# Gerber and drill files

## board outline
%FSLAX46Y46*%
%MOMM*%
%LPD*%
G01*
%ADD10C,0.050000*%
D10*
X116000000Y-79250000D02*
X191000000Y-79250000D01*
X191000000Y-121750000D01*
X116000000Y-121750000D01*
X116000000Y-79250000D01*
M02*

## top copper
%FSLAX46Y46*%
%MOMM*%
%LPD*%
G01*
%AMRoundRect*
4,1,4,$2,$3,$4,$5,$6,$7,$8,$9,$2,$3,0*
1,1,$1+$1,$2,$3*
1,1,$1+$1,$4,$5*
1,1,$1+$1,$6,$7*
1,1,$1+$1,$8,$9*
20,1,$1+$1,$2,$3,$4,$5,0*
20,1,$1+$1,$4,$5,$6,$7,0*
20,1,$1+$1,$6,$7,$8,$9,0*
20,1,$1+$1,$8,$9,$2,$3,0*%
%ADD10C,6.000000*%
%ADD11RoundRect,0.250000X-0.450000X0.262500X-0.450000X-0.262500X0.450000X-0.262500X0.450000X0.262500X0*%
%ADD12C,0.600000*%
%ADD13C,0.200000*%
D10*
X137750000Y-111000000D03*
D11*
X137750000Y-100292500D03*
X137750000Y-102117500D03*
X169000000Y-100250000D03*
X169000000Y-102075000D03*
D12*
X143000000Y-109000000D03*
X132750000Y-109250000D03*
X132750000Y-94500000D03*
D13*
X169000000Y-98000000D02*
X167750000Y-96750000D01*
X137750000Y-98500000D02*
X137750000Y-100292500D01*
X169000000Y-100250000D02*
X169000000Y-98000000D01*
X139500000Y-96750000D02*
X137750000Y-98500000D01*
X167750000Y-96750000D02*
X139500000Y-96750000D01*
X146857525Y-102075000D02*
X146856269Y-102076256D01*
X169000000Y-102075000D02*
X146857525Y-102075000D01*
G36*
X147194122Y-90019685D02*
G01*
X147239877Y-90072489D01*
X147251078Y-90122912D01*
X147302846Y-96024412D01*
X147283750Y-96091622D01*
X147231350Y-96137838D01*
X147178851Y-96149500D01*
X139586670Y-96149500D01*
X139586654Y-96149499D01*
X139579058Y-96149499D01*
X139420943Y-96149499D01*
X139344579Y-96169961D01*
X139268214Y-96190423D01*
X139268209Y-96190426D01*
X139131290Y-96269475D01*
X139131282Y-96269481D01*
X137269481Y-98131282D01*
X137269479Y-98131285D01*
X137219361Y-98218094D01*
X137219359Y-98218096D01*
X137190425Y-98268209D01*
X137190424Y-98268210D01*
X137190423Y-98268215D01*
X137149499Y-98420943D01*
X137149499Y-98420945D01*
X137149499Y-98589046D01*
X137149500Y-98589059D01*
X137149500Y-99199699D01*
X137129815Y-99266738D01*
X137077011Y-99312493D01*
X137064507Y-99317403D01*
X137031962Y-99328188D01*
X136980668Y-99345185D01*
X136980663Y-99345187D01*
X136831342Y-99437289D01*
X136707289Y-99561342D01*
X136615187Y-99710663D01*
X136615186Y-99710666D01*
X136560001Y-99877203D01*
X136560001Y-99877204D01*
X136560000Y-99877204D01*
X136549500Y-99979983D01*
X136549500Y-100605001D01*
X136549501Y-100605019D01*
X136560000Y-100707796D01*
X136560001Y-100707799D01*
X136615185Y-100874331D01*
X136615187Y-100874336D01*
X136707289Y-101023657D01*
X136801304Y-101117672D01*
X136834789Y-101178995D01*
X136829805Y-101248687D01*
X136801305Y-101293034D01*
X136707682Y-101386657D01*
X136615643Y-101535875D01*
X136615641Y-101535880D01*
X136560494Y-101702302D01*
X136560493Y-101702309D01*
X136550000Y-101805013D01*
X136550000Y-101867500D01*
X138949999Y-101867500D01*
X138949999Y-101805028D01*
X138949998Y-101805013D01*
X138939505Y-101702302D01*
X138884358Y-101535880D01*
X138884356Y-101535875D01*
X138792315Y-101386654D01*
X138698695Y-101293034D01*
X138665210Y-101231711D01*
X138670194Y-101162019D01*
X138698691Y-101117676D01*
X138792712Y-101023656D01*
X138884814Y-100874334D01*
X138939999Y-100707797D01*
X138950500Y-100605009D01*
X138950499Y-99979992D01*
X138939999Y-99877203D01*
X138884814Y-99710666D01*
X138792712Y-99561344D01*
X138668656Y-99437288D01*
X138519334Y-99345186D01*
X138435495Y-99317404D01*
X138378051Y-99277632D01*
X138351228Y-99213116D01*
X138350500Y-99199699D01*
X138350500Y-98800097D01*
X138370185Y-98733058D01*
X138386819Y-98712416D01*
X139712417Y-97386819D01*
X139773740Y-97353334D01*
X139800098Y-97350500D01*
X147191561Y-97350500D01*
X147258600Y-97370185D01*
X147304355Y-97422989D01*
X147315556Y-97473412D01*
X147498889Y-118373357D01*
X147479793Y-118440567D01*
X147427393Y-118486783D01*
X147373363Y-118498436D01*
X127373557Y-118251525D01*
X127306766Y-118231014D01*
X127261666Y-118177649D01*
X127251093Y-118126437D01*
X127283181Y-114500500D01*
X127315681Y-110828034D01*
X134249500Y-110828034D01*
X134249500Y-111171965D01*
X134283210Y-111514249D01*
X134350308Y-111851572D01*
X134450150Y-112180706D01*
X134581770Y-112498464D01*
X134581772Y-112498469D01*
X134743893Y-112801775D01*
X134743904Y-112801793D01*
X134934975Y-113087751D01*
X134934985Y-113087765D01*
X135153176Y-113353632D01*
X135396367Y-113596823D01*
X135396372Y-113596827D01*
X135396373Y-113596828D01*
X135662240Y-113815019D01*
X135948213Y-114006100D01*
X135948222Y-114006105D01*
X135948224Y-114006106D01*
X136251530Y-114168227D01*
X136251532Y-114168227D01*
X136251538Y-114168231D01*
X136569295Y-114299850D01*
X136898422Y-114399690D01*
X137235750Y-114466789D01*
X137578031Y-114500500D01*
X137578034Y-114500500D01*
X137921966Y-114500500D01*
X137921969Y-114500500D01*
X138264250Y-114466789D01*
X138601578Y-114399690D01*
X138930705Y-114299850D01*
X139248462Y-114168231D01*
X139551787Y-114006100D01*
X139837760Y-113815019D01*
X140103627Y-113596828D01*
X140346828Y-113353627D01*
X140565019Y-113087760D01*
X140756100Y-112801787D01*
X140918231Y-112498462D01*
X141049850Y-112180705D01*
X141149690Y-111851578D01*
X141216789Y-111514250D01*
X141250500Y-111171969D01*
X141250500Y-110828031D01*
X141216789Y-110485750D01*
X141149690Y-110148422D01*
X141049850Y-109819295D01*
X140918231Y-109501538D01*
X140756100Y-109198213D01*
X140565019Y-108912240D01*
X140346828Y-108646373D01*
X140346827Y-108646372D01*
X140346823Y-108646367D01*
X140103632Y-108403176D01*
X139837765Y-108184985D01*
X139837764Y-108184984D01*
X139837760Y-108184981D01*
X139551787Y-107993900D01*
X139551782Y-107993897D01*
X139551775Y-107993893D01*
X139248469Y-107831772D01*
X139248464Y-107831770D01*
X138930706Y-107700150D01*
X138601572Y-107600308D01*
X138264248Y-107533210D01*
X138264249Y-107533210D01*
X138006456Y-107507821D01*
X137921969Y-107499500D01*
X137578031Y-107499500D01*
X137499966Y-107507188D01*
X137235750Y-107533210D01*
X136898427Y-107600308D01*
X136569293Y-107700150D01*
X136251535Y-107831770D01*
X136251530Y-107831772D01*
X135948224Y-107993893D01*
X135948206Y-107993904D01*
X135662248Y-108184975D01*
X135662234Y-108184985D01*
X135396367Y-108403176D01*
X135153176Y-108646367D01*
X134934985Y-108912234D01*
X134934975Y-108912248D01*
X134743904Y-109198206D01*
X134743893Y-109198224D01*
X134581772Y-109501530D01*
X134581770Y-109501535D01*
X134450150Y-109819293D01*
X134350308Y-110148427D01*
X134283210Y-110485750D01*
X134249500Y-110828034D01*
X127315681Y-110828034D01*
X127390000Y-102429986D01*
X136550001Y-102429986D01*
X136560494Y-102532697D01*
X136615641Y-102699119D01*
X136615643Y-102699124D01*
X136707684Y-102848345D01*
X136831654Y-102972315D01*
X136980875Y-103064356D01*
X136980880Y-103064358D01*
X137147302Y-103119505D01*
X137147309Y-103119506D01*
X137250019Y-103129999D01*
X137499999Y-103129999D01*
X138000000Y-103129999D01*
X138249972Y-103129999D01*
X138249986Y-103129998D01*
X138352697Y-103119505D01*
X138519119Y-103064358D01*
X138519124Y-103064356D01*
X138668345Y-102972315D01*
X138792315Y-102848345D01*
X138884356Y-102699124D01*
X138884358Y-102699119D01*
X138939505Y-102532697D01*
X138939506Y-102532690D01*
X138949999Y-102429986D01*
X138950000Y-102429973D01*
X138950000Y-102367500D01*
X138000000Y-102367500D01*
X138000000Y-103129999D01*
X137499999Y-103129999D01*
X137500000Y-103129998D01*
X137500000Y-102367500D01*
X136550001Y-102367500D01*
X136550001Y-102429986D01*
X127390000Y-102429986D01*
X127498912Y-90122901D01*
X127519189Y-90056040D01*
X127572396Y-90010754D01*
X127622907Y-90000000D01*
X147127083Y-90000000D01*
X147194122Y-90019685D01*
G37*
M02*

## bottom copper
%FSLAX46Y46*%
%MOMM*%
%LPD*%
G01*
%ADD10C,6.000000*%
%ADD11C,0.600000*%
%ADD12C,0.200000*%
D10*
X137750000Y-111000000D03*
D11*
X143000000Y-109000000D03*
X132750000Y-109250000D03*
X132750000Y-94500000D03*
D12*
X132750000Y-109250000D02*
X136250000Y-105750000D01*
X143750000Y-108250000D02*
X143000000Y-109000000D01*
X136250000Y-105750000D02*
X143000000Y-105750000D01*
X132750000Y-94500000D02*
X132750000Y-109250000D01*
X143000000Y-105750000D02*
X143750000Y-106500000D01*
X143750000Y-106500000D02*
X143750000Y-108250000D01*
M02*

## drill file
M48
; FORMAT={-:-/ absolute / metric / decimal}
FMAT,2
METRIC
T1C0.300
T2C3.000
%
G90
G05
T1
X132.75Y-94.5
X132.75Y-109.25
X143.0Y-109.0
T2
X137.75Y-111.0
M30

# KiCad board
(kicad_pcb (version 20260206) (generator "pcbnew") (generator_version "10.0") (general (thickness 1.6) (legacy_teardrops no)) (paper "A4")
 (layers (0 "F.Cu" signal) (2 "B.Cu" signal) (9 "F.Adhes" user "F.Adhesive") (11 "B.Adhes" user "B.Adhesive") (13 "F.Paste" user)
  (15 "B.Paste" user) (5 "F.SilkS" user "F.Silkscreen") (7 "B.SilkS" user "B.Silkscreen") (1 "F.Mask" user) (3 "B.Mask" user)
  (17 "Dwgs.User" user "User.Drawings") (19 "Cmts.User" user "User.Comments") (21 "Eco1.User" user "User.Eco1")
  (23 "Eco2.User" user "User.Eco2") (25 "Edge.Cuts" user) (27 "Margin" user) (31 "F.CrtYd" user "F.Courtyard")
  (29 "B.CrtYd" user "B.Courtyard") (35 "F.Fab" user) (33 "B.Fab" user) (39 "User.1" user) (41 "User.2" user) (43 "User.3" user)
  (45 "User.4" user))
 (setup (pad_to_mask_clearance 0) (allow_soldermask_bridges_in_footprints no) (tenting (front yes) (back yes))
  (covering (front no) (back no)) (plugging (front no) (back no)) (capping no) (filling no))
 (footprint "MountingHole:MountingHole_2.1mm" (layer "F.Cu") (at 137.75 111)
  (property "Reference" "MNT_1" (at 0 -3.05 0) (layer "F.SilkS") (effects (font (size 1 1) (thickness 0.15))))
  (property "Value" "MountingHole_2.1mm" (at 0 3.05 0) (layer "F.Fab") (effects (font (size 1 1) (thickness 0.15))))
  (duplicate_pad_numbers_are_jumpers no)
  (pad "" np_thru_hole circle (at 0 0) (size 6 6) (drill 3) (layers "*.Cu" "*.Mask")))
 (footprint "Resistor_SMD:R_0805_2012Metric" (layer "F.Cu") (at 137.75 101.205 -90)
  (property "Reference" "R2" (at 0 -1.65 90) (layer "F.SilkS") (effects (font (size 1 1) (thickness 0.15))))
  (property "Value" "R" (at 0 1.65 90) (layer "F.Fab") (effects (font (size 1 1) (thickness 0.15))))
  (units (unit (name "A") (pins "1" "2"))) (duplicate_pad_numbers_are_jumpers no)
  (pad "1" smd roundrect (at -0.9125 0 270) (size 1.025 1.4) (layers "F.Cu" "F.Mask" "F.Paste") (roundrect_rratio 0.243902) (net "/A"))
  (pad "2" smd roundrect (at 0.9125 0 270) (size 1.025 1.4) (layers "F.Cu" "F.Mask" "F.Paste") (roundrect_rratio 0.243902) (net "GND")))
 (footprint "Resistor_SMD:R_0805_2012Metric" (layer "F.Cu") (at 169 101.1625 -90)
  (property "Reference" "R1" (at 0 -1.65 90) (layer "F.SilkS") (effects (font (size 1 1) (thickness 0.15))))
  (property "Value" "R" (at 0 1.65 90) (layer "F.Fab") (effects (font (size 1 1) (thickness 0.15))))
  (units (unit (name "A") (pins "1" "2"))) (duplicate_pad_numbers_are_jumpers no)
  (pad "1" smd roundrect (at -0.9125 0 270) (size 1.025 1.4) (layers "F.Cu" "F.Mask" "F.Paste") (roundrect_rratio 0.243902) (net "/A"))
  (pad "2" smd roundrect (at 0.9125 0 270) (size 1.025 1.4) (layers "F.Cu" "F.Mask" "F.Paste") (roundrect_rratio 0.243902) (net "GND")))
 (gr_rect (start 116 79.25) (end 191 121.75) (stroke (width 0.05) (type default)) (fill no) (layer "Edge.Cuts"))
 (segment (start 169 98) (end 167.75 96.75) (width 0.2) (layer "F.Cu") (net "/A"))
 (segment (start 137.75 98.5) (end 137.75 100.2925) (width 0.2) (layer "F.Cu") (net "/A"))
 (segment (start 169 100.25) (end 169 98) (width 0.2) (layer "F.Cu") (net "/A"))
 (segment (start 139.5 96.75) (end 137.75 98.5) (width 0.2) (layer "F.Cu") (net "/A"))
 (segment (start 167.75 96.75) (end 139.5 96.75) (width 0.2) (layer "F.Cu") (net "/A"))
 (segment (start 146.857525 102.075) (end 146.856269 102.076256) (width 0.2) (layer "F.Cu") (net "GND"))
 (segment (start 169 102.075) (end 146.857525 102.075) (width 0.2) (layer "F.Cu") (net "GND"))
 (via (at 143 109) (size 0.6) (drill 0.3) (layers "F.Cu" "B.Cu") (free yes) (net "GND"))
 (via (at 132.75 109.25) (size 0.6) (drill 0.3) (layers "F.Cu" "B.Cu") (free yes) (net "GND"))
 (via (at 132.75 94.5) (size 0.6) (drill 0.3) (layers "F.Cu" "B.Cu") (free yes) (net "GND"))
 (segment (start 132.75 109.25) (end 136.25 105.75) (width 0.2) (layer "B.Cu") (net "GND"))
 (segment (start 143.75 108.25) (end 143 109) (width 0.2) (layer "B.Cu") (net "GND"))
 (segment (start 136.25 105.75) (end 143 105.75) (width 0.2) (layer "B.Cu") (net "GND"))
 (segment (start 132.75 94.5) (end 132.75 109.25) (width 0.2) (layer "B.Cu") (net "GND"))
 (segment (start 143 105.75) (end 143.75 106.5) (width 0.2) (layer "B.Cu") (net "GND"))
 (segment (start 143.75 106.5) (end 143.75 108.25) (width 0.2) (layer "B.Cu") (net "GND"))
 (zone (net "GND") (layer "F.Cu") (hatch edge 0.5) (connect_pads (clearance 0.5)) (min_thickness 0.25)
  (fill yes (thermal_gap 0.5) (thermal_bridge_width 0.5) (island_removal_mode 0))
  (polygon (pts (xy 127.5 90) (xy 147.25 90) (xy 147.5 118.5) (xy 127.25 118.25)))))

